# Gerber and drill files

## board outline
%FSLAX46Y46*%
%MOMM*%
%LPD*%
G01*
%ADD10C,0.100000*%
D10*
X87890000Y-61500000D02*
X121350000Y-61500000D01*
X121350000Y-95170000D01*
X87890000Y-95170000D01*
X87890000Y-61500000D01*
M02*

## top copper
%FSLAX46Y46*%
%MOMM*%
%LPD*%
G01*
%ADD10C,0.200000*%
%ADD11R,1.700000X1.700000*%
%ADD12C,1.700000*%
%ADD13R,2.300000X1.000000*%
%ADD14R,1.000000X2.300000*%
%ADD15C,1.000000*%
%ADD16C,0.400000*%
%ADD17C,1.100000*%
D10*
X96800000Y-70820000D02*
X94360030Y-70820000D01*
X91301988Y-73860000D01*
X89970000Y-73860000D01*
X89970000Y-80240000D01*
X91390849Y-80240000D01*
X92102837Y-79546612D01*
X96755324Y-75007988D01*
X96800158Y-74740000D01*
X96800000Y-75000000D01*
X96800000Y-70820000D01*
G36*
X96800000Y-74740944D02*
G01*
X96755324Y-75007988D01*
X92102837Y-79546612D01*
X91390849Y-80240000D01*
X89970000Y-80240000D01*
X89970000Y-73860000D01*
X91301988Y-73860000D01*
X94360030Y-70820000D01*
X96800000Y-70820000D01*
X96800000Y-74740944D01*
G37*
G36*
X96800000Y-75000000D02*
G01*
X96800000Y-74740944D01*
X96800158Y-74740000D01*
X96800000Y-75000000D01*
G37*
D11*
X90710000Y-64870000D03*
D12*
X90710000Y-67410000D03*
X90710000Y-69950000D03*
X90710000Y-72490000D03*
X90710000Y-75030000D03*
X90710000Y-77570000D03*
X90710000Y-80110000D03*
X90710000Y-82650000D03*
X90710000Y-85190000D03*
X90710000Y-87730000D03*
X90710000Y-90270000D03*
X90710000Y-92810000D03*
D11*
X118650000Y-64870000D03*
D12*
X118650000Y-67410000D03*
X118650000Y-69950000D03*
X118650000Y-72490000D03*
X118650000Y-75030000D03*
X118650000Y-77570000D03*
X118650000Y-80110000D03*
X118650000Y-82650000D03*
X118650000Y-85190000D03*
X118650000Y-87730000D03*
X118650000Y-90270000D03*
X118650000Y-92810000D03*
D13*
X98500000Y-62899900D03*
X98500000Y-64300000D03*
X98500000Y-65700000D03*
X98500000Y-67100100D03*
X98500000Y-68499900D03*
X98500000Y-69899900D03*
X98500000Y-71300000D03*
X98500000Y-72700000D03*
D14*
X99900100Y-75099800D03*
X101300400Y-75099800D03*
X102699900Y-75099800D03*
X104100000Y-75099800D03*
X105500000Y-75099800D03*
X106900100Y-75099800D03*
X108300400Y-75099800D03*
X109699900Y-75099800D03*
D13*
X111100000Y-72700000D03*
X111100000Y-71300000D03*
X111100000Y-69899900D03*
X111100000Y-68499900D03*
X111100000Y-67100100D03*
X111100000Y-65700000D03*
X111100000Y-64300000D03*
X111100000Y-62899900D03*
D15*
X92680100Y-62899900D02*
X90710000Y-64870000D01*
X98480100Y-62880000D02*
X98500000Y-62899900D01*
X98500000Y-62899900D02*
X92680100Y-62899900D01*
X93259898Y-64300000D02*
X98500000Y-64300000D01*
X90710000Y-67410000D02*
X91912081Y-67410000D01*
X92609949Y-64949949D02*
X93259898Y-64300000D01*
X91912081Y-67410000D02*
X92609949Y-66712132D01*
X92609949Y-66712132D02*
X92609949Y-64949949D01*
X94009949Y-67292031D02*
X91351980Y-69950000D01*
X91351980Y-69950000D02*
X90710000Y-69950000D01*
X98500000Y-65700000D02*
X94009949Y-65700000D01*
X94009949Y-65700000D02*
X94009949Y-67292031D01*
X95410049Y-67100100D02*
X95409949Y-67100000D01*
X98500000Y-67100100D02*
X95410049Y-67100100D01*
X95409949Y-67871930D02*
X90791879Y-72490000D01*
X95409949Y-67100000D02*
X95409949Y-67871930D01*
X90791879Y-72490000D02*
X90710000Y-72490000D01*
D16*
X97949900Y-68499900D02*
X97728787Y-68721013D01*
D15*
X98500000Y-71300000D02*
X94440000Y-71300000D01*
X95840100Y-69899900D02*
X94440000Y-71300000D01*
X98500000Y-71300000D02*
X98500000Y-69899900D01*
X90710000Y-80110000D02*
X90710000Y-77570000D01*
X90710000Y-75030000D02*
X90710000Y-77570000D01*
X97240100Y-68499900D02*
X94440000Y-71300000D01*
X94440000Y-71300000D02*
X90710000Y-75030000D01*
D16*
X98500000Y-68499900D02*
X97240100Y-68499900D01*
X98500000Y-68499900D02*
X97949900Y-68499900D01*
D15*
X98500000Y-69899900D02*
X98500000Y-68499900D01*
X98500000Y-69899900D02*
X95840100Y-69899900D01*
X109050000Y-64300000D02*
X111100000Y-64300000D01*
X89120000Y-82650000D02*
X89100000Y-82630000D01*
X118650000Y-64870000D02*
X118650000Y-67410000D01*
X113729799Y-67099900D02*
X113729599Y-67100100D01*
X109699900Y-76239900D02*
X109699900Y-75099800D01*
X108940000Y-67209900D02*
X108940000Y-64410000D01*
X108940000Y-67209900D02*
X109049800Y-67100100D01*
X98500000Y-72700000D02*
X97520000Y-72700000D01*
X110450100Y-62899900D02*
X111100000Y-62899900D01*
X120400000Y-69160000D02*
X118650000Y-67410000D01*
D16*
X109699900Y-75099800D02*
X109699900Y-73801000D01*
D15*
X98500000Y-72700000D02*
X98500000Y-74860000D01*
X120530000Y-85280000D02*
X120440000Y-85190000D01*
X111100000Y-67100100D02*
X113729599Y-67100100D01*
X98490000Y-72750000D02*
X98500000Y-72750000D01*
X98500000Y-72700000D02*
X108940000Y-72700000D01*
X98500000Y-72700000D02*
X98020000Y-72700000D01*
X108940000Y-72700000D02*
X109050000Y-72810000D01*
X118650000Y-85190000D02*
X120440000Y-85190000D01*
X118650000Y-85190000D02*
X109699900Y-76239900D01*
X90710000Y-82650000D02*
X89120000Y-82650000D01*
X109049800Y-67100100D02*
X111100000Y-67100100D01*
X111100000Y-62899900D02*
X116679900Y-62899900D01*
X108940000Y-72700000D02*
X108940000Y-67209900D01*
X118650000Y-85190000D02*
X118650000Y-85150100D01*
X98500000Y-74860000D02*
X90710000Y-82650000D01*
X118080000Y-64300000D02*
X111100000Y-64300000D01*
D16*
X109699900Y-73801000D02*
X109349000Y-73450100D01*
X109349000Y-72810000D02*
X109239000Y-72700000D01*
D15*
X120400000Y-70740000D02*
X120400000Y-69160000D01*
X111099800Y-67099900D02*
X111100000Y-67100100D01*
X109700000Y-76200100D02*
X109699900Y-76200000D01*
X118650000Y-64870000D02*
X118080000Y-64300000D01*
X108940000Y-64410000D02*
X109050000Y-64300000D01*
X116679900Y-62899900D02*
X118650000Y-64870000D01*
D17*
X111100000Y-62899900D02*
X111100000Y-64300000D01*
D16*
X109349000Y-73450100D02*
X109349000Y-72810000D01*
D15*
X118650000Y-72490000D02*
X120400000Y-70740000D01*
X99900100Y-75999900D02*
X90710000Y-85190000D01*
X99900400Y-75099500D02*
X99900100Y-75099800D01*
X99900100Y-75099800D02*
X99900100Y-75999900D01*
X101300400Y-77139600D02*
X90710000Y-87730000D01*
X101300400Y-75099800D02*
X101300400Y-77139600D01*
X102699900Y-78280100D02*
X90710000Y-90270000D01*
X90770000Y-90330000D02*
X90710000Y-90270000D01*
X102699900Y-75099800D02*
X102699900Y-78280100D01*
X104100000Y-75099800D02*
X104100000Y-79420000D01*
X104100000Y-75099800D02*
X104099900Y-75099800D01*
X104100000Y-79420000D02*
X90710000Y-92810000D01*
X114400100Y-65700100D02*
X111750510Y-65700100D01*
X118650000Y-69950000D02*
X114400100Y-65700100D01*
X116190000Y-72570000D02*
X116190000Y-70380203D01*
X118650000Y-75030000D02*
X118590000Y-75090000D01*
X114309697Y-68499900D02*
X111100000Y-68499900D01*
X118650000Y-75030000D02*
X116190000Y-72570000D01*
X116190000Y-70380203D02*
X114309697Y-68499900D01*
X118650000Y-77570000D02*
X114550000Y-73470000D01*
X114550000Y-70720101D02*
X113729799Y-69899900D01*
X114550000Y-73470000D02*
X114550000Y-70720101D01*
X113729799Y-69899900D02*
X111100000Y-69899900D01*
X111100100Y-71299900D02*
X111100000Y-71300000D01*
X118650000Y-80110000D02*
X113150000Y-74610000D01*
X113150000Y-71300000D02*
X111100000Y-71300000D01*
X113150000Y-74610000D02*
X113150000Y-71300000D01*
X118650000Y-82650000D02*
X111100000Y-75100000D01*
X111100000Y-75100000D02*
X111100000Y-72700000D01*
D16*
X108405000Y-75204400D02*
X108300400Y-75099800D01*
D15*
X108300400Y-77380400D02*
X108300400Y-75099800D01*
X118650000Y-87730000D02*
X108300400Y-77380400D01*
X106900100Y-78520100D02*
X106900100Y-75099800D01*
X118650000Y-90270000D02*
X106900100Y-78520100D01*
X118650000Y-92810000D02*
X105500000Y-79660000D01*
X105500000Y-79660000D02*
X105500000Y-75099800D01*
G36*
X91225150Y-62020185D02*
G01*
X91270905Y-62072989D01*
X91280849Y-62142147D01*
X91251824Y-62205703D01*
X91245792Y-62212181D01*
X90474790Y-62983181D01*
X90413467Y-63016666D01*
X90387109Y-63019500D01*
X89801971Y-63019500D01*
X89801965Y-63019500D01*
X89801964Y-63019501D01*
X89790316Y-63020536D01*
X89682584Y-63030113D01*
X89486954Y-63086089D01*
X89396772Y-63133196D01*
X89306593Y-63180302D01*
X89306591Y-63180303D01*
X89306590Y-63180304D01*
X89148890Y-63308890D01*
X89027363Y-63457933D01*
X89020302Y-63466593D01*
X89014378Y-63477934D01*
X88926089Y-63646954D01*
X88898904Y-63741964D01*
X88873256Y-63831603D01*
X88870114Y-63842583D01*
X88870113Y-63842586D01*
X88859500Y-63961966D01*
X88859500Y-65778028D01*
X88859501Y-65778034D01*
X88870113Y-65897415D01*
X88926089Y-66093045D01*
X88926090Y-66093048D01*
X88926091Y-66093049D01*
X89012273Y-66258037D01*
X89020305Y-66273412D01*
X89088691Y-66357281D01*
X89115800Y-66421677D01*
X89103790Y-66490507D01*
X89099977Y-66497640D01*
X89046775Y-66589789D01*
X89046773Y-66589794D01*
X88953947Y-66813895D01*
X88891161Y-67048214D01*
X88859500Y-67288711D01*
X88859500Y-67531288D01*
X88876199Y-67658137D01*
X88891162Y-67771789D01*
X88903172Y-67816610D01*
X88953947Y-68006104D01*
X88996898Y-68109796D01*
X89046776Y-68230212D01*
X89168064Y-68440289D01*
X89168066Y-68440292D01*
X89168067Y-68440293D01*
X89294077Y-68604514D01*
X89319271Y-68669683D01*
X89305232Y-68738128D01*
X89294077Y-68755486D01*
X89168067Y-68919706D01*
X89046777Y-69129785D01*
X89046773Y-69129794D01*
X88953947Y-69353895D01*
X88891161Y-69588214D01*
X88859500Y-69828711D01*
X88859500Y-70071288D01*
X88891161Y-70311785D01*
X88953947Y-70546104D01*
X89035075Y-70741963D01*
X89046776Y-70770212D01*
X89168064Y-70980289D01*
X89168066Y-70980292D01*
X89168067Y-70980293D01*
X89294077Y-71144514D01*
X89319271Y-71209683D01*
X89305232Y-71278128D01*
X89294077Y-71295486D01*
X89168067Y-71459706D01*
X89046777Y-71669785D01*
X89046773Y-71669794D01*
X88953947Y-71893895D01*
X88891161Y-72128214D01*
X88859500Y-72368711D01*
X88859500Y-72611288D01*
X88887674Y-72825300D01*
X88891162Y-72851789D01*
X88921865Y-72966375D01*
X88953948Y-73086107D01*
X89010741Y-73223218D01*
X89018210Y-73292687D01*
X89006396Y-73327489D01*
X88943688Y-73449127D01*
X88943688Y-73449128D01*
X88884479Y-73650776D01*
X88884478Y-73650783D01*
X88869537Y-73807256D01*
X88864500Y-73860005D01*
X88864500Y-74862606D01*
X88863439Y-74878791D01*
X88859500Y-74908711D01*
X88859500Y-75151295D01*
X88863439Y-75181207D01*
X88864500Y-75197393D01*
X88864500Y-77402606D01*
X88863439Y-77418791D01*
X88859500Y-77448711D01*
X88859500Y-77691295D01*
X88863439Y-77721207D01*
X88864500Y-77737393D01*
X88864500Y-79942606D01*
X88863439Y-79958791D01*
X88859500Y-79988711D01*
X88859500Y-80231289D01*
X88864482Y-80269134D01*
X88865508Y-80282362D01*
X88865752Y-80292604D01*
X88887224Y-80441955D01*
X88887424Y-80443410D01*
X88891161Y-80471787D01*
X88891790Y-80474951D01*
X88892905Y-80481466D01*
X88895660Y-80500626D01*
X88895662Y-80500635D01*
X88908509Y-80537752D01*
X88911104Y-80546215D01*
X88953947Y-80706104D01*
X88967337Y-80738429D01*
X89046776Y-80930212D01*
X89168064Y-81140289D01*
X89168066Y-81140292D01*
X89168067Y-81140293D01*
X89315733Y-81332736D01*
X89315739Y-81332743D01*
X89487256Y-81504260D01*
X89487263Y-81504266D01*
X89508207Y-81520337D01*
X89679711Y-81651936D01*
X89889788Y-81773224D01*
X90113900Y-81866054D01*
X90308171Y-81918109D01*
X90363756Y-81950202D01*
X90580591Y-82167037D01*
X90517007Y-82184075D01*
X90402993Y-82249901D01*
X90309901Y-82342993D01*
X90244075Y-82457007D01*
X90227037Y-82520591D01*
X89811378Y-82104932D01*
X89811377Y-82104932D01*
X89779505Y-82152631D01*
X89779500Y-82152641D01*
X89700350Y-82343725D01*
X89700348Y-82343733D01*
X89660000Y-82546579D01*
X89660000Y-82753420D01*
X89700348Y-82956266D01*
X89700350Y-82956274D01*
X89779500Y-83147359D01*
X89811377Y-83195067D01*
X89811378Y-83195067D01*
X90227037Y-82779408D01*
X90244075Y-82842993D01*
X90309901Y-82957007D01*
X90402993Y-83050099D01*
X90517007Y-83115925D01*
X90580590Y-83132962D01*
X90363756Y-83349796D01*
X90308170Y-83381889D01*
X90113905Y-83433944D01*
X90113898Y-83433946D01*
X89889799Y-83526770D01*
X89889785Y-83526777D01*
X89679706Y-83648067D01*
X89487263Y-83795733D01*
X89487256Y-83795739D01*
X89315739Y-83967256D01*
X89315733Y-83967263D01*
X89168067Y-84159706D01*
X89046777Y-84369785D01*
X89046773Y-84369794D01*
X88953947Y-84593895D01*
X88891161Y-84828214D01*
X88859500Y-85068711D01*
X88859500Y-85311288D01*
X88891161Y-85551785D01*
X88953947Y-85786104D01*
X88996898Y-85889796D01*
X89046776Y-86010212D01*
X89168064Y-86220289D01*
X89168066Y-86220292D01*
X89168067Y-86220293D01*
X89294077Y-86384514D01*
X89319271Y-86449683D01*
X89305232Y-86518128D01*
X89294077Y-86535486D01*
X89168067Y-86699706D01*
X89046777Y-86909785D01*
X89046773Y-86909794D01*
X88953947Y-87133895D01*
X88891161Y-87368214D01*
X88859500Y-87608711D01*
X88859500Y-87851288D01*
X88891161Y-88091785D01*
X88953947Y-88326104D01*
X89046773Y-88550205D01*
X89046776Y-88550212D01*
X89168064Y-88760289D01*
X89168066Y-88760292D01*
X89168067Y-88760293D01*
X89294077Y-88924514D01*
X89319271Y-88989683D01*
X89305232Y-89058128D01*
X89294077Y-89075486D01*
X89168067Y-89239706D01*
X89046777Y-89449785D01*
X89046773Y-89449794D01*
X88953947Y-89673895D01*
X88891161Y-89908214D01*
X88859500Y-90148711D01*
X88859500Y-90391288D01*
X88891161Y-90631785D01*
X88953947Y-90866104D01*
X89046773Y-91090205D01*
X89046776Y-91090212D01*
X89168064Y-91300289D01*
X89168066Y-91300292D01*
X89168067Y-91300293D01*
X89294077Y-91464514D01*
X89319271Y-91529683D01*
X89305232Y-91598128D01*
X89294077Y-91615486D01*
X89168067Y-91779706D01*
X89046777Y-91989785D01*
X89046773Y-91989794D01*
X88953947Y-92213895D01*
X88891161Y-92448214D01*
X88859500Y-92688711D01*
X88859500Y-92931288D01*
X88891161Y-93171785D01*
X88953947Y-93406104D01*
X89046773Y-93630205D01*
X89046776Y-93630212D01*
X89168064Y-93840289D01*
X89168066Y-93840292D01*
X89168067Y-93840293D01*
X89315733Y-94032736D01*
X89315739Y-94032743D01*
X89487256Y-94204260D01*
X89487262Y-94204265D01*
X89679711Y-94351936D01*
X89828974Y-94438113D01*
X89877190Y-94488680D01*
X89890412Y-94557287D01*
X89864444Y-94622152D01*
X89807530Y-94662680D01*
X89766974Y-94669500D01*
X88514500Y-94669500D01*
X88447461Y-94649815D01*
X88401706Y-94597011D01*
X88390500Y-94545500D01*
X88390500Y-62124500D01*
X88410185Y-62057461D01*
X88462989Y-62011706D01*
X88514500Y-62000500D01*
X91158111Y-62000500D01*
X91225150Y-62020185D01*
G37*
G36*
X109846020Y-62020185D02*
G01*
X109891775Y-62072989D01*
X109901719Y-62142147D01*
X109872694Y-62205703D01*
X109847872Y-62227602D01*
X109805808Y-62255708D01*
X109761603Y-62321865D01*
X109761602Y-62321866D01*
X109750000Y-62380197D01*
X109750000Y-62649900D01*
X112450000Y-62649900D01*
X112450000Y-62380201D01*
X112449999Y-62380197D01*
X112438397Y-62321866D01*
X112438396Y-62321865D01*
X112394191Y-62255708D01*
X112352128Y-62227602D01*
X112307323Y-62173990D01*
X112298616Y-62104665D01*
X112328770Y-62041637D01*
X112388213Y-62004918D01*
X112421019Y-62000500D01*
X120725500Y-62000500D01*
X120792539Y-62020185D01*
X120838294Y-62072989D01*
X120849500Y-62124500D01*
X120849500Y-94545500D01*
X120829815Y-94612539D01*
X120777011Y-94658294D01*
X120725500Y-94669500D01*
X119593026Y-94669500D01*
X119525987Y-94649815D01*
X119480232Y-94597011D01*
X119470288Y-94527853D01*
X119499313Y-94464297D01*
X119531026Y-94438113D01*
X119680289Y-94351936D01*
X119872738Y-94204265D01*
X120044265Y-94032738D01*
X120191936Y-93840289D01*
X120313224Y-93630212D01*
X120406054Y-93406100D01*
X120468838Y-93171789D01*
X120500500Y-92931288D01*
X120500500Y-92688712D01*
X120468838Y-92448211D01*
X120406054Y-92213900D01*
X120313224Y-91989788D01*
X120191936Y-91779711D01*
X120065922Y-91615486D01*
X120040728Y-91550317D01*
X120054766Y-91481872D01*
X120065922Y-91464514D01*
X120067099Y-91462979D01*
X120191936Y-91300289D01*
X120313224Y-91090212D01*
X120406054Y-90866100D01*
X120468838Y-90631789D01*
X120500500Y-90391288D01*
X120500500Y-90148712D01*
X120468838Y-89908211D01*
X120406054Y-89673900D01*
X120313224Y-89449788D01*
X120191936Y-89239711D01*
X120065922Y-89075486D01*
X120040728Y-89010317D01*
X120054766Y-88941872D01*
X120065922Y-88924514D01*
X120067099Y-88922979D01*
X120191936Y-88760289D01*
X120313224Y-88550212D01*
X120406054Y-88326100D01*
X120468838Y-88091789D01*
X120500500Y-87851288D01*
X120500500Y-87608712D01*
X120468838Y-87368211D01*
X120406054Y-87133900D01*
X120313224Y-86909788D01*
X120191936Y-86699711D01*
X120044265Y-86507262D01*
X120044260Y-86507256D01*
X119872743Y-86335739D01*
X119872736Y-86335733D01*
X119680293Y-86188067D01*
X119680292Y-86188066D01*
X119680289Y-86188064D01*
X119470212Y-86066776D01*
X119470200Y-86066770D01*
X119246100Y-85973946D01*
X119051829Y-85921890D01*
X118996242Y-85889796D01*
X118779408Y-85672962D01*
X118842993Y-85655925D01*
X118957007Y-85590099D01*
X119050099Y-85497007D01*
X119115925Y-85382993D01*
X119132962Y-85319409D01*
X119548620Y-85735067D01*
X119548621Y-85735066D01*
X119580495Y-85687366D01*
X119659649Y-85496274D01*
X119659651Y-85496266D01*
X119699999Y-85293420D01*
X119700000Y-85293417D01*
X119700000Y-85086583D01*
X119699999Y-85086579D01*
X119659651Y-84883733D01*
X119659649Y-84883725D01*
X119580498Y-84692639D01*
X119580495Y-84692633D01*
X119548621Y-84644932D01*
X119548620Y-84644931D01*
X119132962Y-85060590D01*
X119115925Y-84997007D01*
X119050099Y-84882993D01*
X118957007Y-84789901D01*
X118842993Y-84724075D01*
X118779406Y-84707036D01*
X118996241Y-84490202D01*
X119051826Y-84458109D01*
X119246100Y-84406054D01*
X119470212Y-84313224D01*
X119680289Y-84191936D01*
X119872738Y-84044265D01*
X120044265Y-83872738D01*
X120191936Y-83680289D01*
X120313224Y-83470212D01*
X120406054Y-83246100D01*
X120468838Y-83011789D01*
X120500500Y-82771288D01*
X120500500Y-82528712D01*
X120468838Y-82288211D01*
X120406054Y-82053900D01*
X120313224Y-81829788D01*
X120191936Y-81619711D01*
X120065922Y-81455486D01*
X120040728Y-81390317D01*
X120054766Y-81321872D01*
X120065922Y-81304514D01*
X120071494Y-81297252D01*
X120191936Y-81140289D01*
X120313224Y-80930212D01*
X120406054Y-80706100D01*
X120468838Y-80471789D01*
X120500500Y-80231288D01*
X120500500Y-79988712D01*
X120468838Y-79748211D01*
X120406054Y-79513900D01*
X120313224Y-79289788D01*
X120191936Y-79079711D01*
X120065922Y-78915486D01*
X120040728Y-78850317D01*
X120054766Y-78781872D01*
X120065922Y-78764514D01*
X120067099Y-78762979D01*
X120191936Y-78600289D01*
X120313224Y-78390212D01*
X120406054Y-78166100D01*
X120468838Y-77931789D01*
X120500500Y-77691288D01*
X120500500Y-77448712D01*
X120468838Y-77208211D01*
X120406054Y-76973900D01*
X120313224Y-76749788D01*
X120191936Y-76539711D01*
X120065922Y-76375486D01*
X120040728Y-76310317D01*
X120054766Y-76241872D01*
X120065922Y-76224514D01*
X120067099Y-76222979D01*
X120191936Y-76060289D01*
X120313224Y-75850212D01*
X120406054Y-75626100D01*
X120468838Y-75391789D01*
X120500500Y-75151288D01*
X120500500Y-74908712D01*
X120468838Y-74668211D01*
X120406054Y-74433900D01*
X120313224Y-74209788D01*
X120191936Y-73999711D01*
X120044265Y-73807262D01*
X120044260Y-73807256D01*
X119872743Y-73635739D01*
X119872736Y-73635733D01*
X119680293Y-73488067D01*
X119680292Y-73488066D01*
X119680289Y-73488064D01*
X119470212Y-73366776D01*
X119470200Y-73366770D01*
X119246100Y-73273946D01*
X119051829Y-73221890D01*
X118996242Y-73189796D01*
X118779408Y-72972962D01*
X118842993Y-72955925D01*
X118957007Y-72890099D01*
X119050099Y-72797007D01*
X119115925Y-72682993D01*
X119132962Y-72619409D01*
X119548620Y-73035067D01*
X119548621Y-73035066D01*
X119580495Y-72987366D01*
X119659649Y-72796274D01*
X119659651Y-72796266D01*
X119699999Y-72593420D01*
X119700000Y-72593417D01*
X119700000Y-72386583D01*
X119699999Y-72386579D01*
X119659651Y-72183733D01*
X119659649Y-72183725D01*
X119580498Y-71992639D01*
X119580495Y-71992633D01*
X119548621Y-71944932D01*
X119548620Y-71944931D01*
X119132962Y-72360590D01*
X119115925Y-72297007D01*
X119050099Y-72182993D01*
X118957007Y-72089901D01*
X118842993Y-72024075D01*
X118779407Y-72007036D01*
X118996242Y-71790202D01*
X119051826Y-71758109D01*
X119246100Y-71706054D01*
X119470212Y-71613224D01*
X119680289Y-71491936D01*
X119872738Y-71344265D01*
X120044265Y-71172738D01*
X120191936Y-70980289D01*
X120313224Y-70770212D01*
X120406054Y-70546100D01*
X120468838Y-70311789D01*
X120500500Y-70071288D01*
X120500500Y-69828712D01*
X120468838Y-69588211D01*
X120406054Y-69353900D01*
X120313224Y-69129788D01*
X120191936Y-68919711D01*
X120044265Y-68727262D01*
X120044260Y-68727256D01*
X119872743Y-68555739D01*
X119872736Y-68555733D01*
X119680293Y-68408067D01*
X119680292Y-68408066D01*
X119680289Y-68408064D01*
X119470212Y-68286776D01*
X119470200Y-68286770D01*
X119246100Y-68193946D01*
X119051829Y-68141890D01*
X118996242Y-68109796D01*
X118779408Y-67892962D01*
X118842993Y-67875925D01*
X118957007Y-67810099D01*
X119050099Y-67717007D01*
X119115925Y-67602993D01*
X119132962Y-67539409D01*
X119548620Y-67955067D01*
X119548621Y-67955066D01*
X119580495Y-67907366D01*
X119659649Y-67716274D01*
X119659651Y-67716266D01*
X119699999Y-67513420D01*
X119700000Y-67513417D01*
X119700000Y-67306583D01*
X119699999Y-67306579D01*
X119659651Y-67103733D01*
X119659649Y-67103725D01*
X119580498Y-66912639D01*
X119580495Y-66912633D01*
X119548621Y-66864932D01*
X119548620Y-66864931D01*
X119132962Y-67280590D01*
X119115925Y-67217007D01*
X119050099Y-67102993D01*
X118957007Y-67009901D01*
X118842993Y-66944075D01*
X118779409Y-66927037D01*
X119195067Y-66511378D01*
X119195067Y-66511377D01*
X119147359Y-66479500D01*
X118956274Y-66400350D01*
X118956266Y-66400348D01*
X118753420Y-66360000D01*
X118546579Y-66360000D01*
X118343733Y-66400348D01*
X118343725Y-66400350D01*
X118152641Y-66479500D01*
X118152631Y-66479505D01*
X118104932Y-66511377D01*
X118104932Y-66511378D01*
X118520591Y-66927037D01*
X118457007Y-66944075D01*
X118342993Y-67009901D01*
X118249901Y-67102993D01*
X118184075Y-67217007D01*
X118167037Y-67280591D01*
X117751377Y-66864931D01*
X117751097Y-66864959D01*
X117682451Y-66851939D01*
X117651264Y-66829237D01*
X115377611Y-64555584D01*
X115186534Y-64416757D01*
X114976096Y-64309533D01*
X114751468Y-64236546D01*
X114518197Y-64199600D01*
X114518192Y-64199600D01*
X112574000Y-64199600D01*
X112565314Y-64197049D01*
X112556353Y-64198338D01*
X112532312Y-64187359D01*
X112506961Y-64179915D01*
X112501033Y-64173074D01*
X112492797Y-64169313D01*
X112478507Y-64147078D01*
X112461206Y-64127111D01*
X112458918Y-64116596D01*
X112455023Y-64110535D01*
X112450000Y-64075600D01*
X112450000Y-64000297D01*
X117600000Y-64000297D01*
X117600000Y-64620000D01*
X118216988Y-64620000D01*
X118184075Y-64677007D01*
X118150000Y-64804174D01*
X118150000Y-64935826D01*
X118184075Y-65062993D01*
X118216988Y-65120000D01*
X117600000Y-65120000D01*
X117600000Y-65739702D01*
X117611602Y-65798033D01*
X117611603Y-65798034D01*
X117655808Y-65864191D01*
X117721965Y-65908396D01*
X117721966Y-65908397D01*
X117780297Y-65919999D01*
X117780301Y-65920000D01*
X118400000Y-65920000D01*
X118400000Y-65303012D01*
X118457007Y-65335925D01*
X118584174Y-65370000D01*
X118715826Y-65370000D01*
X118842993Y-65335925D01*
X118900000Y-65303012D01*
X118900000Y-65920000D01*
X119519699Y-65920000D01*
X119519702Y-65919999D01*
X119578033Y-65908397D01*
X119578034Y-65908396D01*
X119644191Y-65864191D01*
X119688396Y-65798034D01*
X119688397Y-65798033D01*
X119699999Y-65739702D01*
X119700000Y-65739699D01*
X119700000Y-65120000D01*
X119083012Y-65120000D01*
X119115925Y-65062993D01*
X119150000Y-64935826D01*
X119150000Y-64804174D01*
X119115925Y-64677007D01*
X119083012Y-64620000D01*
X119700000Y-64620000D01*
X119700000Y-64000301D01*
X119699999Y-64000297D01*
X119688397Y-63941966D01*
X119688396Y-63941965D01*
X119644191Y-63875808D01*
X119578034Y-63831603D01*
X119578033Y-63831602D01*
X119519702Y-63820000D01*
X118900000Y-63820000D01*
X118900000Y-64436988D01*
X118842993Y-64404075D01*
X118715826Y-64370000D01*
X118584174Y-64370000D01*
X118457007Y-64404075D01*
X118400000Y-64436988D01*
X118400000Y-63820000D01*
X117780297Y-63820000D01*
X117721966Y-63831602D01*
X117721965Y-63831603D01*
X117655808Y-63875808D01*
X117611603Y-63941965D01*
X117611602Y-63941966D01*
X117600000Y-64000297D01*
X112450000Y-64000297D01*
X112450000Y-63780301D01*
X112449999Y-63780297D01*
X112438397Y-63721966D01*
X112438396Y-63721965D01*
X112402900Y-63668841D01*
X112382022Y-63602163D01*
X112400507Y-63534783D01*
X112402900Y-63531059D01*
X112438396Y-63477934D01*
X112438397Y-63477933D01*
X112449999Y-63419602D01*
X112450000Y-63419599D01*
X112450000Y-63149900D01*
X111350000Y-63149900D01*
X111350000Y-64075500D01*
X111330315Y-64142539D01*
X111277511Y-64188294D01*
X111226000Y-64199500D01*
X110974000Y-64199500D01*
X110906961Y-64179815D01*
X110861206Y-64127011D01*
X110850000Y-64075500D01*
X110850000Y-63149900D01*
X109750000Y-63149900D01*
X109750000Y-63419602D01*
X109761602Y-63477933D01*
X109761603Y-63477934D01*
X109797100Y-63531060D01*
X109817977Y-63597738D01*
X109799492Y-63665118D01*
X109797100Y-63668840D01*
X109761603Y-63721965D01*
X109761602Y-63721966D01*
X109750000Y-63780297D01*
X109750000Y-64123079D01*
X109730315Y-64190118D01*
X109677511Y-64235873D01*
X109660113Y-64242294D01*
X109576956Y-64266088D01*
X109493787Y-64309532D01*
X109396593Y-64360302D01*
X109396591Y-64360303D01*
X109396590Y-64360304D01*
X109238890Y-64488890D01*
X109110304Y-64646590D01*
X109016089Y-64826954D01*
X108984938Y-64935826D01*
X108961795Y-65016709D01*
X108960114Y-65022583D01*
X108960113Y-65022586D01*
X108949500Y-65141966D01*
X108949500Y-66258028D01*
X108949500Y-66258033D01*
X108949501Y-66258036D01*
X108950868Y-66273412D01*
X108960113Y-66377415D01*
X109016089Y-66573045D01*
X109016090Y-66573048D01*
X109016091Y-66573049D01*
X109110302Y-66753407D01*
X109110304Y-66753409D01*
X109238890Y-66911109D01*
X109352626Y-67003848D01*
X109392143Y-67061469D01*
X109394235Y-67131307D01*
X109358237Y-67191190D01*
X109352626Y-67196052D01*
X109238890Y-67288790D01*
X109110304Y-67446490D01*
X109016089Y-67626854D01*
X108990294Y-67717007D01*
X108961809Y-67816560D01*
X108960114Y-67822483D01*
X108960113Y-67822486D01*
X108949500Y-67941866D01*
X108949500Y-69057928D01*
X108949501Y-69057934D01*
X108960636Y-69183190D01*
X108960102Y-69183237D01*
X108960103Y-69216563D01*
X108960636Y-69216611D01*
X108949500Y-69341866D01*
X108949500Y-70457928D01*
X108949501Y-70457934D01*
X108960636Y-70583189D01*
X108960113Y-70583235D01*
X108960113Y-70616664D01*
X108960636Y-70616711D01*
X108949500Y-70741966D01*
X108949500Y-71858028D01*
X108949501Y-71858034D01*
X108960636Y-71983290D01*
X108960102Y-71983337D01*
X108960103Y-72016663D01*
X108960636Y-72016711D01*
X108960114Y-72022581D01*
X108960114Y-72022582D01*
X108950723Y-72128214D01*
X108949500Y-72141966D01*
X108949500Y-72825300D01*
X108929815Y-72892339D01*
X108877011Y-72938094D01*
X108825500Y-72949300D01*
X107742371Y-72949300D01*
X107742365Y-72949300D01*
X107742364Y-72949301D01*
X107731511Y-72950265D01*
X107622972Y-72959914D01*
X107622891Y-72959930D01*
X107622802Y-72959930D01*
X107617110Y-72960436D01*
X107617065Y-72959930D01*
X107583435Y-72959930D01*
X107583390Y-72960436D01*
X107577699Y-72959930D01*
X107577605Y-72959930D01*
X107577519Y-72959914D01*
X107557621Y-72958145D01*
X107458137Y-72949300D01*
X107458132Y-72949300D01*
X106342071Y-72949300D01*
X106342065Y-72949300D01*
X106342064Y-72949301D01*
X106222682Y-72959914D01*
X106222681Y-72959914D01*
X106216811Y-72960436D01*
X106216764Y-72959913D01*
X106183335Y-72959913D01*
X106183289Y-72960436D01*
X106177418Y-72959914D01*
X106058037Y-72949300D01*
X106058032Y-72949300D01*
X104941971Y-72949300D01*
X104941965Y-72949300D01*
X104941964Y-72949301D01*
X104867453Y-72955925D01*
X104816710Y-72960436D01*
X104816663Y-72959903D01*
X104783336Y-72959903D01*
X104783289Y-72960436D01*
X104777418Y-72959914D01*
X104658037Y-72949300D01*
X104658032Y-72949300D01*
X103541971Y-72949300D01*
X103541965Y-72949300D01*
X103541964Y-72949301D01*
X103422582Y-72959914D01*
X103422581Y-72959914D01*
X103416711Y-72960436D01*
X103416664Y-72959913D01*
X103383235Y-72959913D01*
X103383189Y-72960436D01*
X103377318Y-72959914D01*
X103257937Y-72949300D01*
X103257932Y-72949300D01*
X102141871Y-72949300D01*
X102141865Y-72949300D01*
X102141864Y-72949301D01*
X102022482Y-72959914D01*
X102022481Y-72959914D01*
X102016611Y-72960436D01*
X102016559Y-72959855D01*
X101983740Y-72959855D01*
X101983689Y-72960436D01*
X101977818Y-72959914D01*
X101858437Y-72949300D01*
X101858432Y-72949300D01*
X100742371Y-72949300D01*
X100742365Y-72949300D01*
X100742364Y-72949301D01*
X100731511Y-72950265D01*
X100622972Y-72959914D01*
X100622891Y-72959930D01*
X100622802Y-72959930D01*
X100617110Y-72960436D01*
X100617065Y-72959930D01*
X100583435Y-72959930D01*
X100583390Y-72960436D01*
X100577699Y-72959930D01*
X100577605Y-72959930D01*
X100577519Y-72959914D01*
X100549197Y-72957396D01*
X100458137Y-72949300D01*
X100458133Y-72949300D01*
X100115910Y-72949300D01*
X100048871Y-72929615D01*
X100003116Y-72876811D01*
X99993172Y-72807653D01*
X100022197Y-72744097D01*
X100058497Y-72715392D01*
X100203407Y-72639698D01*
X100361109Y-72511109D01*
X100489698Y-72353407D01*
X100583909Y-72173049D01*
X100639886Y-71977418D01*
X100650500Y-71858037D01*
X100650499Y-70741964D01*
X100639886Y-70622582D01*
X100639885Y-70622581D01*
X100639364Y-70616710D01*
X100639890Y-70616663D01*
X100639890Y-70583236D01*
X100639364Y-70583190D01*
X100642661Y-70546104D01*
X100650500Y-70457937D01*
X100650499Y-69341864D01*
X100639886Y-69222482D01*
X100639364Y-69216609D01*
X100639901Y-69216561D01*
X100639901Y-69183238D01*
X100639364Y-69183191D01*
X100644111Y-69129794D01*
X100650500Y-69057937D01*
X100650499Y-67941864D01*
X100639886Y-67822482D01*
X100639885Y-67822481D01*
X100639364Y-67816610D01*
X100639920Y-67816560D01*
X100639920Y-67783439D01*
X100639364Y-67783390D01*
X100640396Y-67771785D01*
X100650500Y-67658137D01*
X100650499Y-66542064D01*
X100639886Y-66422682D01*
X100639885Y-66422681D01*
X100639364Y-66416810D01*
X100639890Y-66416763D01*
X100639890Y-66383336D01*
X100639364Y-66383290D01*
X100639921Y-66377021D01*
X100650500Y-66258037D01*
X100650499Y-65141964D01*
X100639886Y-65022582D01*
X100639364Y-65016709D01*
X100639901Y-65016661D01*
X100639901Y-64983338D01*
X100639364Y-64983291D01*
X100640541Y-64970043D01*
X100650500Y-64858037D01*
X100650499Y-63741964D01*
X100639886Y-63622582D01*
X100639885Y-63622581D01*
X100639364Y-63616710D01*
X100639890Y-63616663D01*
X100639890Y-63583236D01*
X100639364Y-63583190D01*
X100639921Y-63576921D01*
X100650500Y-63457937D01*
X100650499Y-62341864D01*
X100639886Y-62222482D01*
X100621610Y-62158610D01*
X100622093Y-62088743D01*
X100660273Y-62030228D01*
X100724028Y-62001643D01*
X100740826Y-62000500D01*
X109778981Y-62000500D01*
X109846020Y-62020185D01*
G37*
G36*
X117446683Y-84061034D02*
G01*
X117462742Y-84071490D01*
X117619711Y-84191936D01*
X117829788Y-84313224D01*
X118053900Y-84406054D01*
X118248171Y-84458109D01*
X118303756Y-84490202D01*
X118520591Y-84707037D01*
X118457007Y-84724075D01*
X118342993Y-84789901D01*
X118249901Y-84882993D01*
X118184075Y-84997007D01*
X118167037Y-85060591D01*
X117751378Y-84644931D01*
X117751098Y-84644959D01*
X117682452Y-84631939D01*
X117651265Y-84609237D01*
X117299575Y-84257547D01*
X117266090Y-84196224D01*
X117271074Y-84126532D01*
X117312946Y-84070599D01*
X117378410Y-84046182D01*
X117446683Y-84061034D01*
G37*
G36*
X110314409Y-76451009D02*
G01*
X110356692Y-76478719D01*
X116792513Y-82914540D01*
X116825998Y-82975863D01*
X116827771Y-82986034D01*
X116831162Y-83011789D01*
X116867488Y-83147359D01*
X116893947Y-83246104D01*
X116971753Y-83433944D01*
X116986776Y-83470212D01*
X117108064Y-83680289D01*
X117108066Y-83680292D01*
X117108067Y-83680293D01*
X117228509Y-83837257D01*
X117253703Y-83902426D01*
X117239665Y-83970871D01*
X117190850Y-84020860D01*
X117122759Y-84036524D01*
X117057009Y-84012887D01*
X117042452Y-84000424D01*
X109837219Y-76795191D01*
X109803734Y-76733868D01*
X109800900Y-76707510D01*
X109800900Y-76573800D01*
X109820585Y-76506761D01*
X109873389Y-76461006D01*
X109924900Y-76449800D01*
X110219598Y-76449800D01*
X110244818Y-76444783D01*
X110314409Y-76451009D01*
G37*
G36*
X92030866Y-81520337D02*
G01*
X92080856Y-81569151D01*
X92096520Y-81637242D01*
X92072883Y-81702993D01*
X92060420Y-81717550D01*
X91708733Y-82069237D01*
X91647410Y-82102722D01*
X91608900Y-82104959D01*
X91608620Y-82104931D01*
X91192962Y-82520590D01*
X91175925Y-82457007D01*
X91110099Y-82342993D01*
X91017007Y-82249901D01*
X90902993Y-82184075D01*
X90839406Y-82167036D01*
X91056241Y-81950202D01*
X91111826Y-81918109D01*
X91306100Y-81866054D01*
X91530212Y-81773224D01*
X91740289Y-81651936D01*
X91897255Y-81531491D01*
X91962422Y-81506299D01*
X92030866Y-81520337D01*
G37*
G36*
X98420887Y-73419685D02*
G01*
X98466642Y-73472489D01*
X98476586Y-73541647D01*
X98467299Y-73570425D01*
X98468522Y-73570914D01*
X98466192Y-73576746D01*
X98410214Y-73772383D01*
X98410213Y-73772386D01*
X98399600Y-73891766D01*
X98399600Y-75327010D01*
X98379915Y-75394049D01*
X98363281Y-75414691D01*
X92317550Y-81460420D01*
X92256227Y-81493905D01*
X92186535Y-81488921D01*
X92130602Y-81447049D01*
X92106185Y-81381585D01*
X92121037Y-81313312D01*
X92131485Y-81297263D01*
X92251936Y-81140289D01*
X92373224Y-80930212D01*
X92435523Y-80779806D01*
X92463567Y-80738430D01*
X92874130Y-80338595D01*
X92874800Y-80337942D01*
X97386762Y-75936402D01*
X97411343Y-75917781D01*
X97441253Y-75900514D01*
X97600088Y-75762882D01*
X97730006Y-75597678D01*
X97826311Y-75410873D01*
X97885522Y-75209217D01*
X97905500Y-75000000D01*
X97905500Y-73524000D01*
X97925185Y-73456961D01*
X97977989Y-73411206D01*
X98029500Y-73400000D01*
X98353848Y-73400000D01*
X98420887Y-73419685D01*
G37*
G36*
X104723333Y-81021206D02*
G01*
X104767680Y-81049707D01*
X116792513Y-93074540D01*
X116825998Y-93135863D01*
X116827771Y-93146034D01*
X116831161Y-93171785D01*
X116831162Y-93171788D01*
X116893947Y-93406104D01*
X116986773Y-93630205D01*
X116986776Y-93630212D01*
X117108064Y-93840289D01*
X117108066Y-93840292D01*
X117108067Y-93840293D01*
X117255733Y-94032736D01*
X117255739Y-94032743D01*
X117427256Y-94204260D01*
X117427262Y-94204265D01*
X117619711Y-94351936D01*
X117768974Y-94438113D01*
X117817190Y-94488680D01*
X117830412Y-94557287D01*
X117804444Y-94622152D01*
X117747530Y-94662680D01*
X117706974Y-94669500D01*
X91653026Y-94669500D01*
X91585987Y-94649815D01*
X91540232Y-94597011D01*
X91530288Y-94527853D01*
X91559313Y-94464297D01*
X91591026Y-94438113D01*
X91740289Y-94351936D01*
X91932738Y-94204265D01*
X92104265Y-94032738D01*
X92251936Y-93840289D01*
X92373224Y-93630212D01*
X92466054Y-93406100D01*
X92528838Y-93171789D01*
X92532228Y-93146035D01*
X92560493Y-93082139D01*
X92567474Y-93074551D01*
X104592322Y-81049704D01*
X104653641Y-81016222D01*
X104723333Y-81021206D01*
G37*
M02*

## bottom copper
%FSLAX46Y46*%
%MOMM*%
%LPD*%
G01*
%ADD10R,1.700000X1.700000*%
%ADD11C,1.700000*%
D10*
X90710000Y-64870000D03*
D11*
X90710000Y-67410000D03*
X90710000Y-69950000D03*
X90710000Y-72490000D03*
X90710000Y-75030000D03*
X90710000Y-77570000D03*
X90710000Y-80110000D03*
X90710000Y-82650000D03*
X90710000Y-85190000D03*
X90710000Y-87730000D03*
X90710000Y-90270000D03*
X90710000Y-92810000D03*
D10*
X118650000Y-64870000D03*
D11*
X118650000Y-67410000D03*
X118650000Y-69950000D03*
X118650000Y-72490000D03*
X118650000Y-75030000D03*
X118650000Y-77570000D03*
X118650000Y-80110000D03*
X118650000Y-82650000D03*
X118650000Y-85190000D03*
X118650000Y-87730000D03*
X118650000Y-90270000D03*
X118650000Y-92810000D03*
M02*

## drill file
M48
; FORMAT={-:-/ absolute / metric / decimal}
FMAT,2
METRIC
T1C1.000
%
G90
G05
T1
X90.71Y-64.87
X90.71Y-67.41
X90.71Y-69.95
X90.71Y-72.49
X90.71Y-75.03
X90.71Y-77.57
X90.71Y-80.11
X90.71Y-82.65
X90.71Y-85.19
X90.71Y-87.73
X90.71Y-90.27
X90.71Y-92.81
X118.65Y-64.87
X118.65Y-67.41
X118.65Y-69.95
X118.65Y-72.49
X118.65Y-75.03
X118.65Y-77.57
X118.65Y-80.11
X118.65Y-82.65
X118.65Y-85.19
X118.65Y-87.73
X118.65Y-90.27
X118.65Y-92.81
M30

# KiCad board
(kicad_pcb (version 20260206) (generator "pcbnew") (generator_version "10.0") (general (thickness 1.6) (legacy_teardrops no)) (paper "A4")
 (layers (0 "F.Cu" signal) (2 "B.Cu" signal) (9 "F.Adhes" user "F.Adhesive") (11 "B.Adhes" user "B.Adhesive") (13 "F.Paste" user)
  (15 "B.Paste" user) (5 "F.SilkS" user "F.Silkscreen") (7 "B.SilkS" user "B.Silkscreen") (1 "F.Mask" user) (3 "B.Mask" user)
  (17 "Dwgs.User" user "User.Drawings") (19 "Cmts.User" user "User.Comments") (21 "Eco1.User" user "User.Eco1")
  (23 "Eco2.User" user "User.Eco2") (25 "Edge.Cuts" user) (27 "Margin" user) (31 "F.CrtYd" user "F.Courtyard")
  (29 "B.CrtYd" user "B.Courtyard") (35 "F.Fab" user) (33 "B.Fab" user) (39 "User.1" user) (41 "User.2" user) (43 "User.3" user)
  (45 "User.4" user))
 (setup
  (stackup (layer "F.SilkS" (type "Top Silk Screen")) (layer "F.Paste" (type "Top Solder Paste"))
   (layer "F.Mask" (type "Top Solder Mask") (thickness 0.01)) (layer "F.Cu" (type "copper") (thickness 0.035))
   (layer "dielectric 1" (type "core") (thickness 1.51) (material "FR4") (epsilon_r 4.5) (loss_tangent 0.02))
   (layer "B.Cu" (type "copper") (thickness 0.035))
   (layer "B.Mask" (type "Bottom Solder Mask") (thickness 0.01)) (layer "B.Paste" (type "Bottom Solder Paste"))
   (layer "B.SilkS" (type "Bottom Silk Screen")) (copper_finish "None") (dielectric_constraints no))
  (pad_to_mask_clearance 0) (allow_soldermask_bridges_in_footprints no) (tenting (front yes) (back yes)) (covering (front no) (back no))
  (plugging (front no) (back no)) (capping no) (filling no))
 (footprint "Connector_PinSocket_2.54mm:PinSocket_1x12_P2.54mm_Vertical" (layer "F.Cu") (at 90.71 64.87)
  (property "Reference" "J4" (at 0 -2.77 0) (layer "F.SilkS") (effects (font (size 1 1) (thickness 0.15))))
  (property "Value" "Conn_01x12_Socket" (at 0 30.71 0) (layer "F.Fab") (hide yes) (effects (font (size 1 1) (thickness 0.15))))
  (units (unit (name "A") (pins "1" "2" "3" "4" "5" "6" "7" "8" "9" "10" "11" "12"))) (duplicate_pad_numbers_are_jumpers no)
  (pad "1" thru_hole rect (at 0 0) (size 1.7 1.7) (drill 1) (layers "*.Cu" "*.Mask") (remove_unused_layers no) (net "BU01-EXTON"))
  (pad "2" thru_hole circle (at 0 2.54) (size 1.7 1.7) (drill 1) (layers "*.Cu" "*.Mask") (remove_unused_layers no) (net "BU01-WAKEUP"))
  (pad "3" thru_hole circle (at 0 5.08) (size 1.7 1.7) (drill 1) (layers "*.Cu" "*.Mask") (remove_unused_layers no) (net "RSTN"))
  (pad "4" thru_hole circle (at 0 7.62) (size 1.7 1.7) (drill 1) (layers "*.Cu" "*.Mask") (remove_unused_layers no) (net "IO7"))
  (pad "5" thru_hole circle (at 0 10.16) (size 1.7 1.7) (drill 1) (layers "*.Cu" "*.Mask") (remove_unused_layers no) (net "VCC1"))
  (pad "6" thru_hole circle (at 0 12.7) (size 1.7 1.7) (drill 1) (layers "*.Cu" "*.Mask") (remove_unused_layers no) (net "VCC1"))
  (pad "7" thru_hole circle (at 0 15.24) (size 1.7 1.7) (drill 1) (layers "*.Cu" "*.Mask") (remove_unused_layers no) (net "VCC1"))
  (pad "8" thru_hole circle (at 0 17.78) (size 1.7 1.7) (drill 1) (layers "*.Cu" "*.Mask") (remove_unused_layers no) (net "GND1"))
  (pad "9" thru_hole circle (at 0 20.32) (size 1.7 1.7) (drill 1) (layers "*.Cu" "*.Mask") (remove_unused_layers no) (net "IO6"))
  (pad "10" thru_hole circle (at 0 22.86) (size 1.7 1.7) (drill 1) (layers "*.Cu" "*.Mask") (remove_unused_layers no) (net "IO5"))
  (pad "11" thru_hole circle (at 0 25.4) (size 1.7 1.7) (drill 1) (layers "*.Cu" "*.Mask") (remove_unused_layers no) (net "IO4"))
  (pad "12" thru_hole circle (at 0 27.94) (size 1.7 1.7) (drill 1) (layers "*.Cu" "*.Mask") (remove_unused_layers no) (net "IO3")))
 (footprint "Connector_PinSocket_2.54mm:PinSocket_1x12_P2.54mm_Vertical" (layer "F.Cu") (at 118.65 64.87)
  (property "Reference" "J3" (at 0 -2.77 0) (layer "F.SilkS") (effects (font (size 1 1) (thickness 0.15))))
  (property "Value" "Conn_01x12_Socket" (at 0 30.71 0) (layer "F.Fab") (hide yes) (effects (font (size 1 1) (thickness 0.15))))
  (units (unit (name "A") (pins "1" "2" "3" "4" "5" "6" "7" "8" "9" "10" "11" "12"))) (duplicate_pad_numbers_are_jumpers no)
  (pad "1" thru_hole rect (at 0 0) (size 1.7 1.7) (drill 1) (layers "*.Cu" "*.Mask") (remove_unused_layers no) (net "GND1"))
  (pad "2" thru_hole circle (at 0 2.54) (size 1.7 1.7) (drill 1) (layers "*.Cu" "*.Mask") (remove_unused_layers no) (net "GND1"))
  (pad "3" thru_hole circle (at 0 5.08) (size 1.7 1.7) (drill 1) (layers "*.Cu" "*.Mask") (remove_unused_layers no) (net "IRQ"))
  (pad "4" thru_hole circle (at 0 7.62) (size 1.7 1.7) (drill 1) (layers "*.Cu" "*.Mask") (remove_unused_layers no) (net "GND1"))
  (pad "5" thru_hole circle (at 0 10.16) (size 1.7 1.7) (drill 1) (layers "*.Cu" "*.Mask") (remove_unused_layers no) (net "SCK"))
  (pad "6" thru_hole circle (at 0 12.7) (size 1.7 1.7) (drill 1) (layers "*.Cu" "*.Mask") (remove_unused_layers no) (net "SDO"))
  (pad "7" thru_hole circle (at 0 15.24) (size 1.7 1.7) (drill 1) (layers "*.Cu" "*.Mask") (remove_unused_layers no) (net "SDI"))
  (pad "8" thru_hole circle (at 0 17.78) (size 1.7 1.7) (drill 1) (layers "*.Cu" "*.Mask") (remove_unused_layers no) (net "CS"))
  (pad "9" thru_hole circle (at 0 20.32) (size 1.7 1.7) (drill 1) (layers "*.Cu" "*.Mask") (remove_unused_layers no) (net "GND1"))
  (pad "10" thru_hole circle (at 0 22.86) (size 1.7 1.7) (drill 1) (layers "*.Cu" "*.Mask") (remove_unused_layers no) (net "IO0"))
  (pad "11" thru_hole circle (at 0 25.4) (size 1.7 1.7) (drill 1) (layers "*.Cu" "*.Mask") (remove_unused_layers no) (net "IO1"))
  (pad "12" thru_hole circle (at 0 27.94) (size 1.7 1.7) (drill 1) (layers "*.Cu" "*.Mask") (remove_unused_layers no) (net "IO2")))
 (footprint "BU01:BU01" (layer "F.Cu") (at 104.8 69)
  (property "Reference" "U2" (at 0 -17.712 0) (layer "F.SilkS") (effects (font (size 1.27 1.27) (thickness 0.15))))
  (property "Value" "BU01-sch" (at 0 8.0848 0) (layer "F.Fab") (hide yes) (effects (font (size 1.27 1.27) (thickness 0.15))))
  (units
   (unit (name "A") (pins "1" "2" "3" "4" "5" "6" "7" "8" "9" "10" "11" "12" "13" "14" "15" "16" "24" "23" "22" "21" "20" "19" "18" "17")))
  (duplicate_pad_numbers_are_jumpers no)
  (pad "1" smd rect (at -6.3 -6.1001) (size 2.3 1) (layers "F.Cu" "F.Mask" "F.Paste") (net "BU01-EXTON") (solder_mask_margin 0.0508)
   (solder_paste_margin 0) (thermal_bridge_angle 0))
  (pad "2" smd rect (at -6.3 -4.7) (size 2.3 1) (layers "F.Cu" "F.Mask" "F.Paste") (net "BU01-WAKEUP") (solder_mask_margin 0.0508)
   (solder_paste_margin 0) (thermal_bridge_angle 0))
  (pad "3" smd rect (at -6.3 -3.3) (size 2.3 1) (layers "F.Cu" "F.Mask" "F.Paste") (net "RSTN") (solder_mask_margin 0.0508)
   (solder_paste_margin 0) (thermal_bridge_angle 0))
  (pad "4" smd rect (at -6.3 -1.8999) (size 2.3 1) (layers "F.Cu" "F.Mask" "F.Paste") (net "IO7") (solder_mask_margin 0.0508)
   (solder_paste_margin 0) (thermal_bridge_angle 0))
  (pad "5" smd rect (at -6.3 -0.5001) (size 2.3 1) (layers "F.Cu" "F.Mask" "F.Paste") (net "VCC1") (solder_mask_margin 0.0508)
   (solder_paste_margin 0) (thermal_bridge_angle 0))
  (pad "6" smd rect (at -6.3 0.8999) (size 2.3 1) (layers "F.Cu" "F.Mask" "F.Paste") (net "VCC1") (solder_mask_margin 0.0508)
   (solder_paste_margin 0) (thermal_bridge_angle 0))
  (pad "7" smd rect (at -6.3 2.3) (size 2.3 1) (layers "F.Cu" "F.Mask" "F.Paste") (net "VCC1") (solder_mask_margin 0.0508)
   (solder_paste_margin 0) (thermal_bridge_angle 0))
  (pad "8" smd rect (at -6.3 3.7) (size 2.3 1) (layers "F.Cu" "F.Mask" "F.Paste") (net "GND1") (solder_mask_margin 0.0508)
   (solder_paste_margin 0) (thermal_bridge_angle 0))
  (pad "9" smd rect (at -4.8999 6.0998) (size 1 2.3) (layers "F.Cu" "F.Mask" "F.Paste") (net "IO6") (solder_mask_margin 0.0508)
   (solder_paste_margin 0) (thermal_bridge_angle 0))
  (pad "10" smd rect (at -3.4996 6.0998) (size 1 2.3) (layers "F.Cu" "F.Mask" "F.Paste") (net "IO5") (solder_mask_margin 0.0508)
   (solder_paste_margin 0) (thermal_bridge_angle 0))
  (pad "11" smd rect (at -2.1001 6.0998) (size 1 2.3) (layers "F.Cu" "F.Mask" "F.Paste") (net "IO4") (solder_mask_margin 0.0508)
   (solder_paste_margin 0) (thermal_bridge_angle 0))
  (pad "12" smd rect (at -0.7 6.0998) (size 1 2.3) (layers "F.Cu" "F.Mask" "F.Paste") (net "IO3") (solder_mask_margin 0.0508)
   (solder_paste_margin 0) (thermal_bridge_angle 0))
  (pad "13" smd rect (at 0.7 6.0998) (size 1 2.3) (layers "F.Cu" "F.Mask" "F.Paste") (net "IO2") (solder_mask_margin 0.0508)
   (solder_paste_margin 0) (thermal_bridge_angle 0))
  (pad "14" smd rect (at 2.1001 6.0998) (size 1 2.3) (layers "F.Cu" "F.Mask" "F.Paste") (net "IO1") (solder_mask_margin 0.0508)
   (solder_paste_margin 0) (thermal_bridge_angle 0))
  (pad "15" smd rect (at 3.5004 6.0998) (size 1 2.3) (layers "F.Cu" "F.Mask" "F.Paste") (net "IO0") (solder_mask_margin 0.0508)
   (solder_paste_margin 0) (thermal_bridge_angle 0))
  (pad "16" smd rect (at 4.8999 6.0998) (size 1 2.3) (layers "F.Cu" "F.Mask" "F.Paste") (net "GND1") (solder_mask_margin 0.0508)
   (solder_paste_margin 0) (thermal_bridge_angle 0))
  (pad "17" smd rect (at 6.3 3.7) (size 2.3 1) (layers "F.Cu" "F.Mask" "F.Paste") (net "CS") (solder_mask_margin 0.0508)
   (solder_paste_margin 0) (thermal_bridge_angle 0))
  (pad "18" smd rect (at 6.3 2.3) (size 2.3 1) (layers "F.Cu" "F.Mask" "F.Paste") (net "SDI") (solder_mask_margin 0.0508)
   (solder_paste_margin 0) (thermal_bridge_angle 0))
  (pad "19" smd rect (at 6.3 0.8999) (size 2.3 1) (layers "F.Cu" "F.Mask" "F.Paste") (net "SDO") (solder_mask_margin 0.0508)
   (solder_paste_margin 0) (thermal_bridge_angle 0))
  (pad "20" smd rect (at 6.3 -0.5001) (size 2.3 1) (layers "F.Cu" "F.Mask" "F.Paste") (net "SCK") (solder_mask_margin 0.0508)
   (solder_paste_margin 0) (thermal_bridge_angle 0))
  (pad "21" smd rect (at 6.3 -1.8999) (size 2.3 1) (layers "F.Cu" "F.Mask" "F.Paste") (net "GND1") (solder_mask_margin 0.0508)
   (solder_paste_margin 0) (thermal_bridge_angle 0))
  (pad "22" smd rect (at 6.3 -3.3) (size 2.3 1) (layers "F.Cu" "F.Mask" "F.Paste") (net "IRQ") (solder_mask_margin 0.0508)
   (solder_paste_margin 0) (thermal_bridge_angle 0))
  (pad "23" smd rect (at 6.3 -4.7) (size 2.3 1) (layers "F.Cu" "F.Mask" "F.Paste") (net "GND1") (solder_mask_margin 0.0508)
   (solder_paste_margin 0) (thermal_bridge_angle 0))
  (pad "24" smd rect (at 6.3 -6.1001) (size 2.3 1) (layers "F.Cu" "F.Mask" "F.Paste") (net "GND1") (solder_mask_margin 0.0508)
   (solder_paste_margin 0) (thermal_bridge_angle 0)))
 (gr_poly
  (pts (xy 96.8 70.82) (xy 94.36003 70.82) (xy 91.301988 73.86) (xy 89.97 73.86) (xy 89.97 80.24) (xy 91.390849 80.24)
   (xy 92.102837 79.546612) (xy 96.755324 75.007988) (xy 96.800158 74.74) (xy 96.8 75))
  (stroke (width 0.2) (type solid)) (fill yes) (layer "F.Cu") (net "VCC1"))
 (gr_rect (start 87.89 61.5) (end 121.35 95.17) (stroke (width 0.1) (type solid)) (fill no) (layer "Edge.Cuts"))
 (segment (start 92.6801 62.8999) (end 90.71 64.87) (width 1) (layer "F.Cu") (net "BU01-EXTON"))
 (segment (start 98.4801 62.88) (end 98.5 62.8999) (width 1) (layer "F.Cu") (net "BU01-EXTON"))
 (segment (start 98.5 62.8999) (end 92.6801 62.8999) (width 1) (layer "F.Cu") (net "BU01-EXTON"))
 (segment (start 93.259898 64.3) (end 98.5 64.3) (width 1) (layer "F.Cu") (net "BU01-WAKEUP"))
 (segment (start 90.71 67.41) (end 91.912081 67.41) (width 1) (layer "F.Cu") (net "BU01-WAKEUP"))
 (segment (start 92.609949 64.949949) (end 93.259898 64.3) (width 1) (layer "F.Cu") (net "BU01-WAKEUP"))
 (segment (start 91.912081 67.41) (end 92.609949 66.712132) (width 1) (layer "F.Cu") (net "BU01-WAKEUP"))
 (segment (start 92.609949 66.712132) (end 92.609949 64.949949) (width 1) (layer "F.Cu") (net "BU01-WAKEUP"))
 (segment (start 94.009949 67.292031) (end 91.35198 69.95) (width 1) (layer "F.Cu") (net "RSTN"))
 (segment (start 91.35198 69.95) (end 90.71 69.95) (width 1) (layer "F.Cu") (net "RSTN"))
 (segment (start 98.5 65.7) (end 94.009949 65.7) (width 1) (layer "F.Cu") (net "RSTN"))
 (segment (start 94.009949 65.7) (end 94.009949 67.292031) (width 1) (layer "F.Cu") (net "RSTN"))
 (segment (start 95.410049 67.1001) (end 95.409949 67.1) (width 1) (layer "F.Cu") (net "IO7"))
 (segment (start 98.5 67.1001) (end 95.410049 67.1001) (width 1) (layer "F.Cu") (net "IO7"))
 (segment (start 95.409949 67.87193) (end 90.791879 72.49) (width 1) (layer "F.Cu") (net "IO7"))
 (segment (start 95.409949 67.1) (end 95.409949 67.87193) (width 1) (layer "F.Cu") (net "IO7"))
 (segment (start 90.791879 72.49) (end 90.71 72.49) (width 1) (layer "F.Cu") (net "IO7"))
 (segment (start 97.9499 68.4999) (end 97.728787 68.721013) (width 0.4) (layer "F.Cu") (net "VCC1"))
 (segment (start 98.5 71.3) (end 94.44 71.3) (width 1) (layer "F.Cu") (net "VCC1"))
 (segment (start 95.8401 69.8999) (end 94.44 71.3) (width 1) (layer "F.Cu") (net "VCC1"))
 (segment (start 98.5 71.3) (end 98.5 69.8999) (width 1) (layer "F.Cu") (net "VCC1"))
 (segment (start 90.71 80.11) (end 90.71 77.57) (width 1) (layer "F.Cu") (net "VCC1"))
 (segment (start 90.71 75.03) (end 90.71 77.57) (width 1) (layer "F.Cu") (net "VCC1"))
 (segment (start 97.2401 68.4999) (end 94.44 71.3) (width 1) (layer "F.Cu") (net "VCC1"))
 (segment (start 94.44 71.3) (end 90.71 75.03) (width 1) (layer "F.Cu") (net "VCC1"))
 (segment (start 98.5 68.4999) (end 97.2401 68.4999) (width 0.4) (layer "F.Cu") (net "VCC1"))
 (segment (start 98.5 68.4999) (end 97.9499 68.4999) (width 0.4) (layer "F.Cu") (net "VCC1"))
 (segment (start 98.5 69.8999) (end 98.5 68.4999) (width 1) (layer "F.Cu") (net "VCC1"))
 (segment (start 98.5 69.8999) (end 95.8401 69.8999) (width 1) (layer "F.Cu") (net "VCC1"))
 (segment (start 109.05 64.3) (end 111.1 64.3) (width 1) (layer "F.Cu") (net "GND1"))
 (segment (start 89.12 82.65) (end 89.1 82.63) (width 1) (layer "F.Cu") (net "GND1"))
 (segment (start 118.65 64.87) (end 118.65 67.41) (width 1) (layer "F.Cu") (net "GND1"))
 (segment (start 113.729799 67.0999) (end 113.729599 67.1001) (width 1) (layer "F.Cu") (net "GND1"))
 (segment (start 109.6999 76.2399) (end 109.6999 75.0998) (width 1) (layer "F.Cu") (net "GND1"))
 (segment (start 108.94 67.2099) (end 108.94 64.41) (width 1) (layer "F.Cu") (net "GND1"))
 (segment (start 108.94 67.2099) (end 109.0498 67.1001) (width 1) (layer "F.Cu") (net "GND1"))
 (segment (start 98.5 72.7) (end 97.52 72.7) (width 1) (layer "F.Cu") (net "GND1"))
 (segment (start 110.4501 62.8999) (end 111.1 62.8999) (width 1) (layer "F.Cu") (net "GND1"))
 (segment (start 120.4 69.16) (end 118.65 67.41) (width 1) (layer "F.Cu") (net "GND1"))
 (segment (start 109.6999 75.0998) (end 109.6999 73.801) (width 0.4) (layer "F.Cu") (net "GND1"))
 (segment (start 98.5 72.7) (end 98.5 74.86) (width 1) (layer "F.Cu") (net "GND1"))
 (segment (start 120.53 85.28) (end 120.44 85.19) (width 1) (layer "F.Cu") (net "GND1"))
 (segment (start 111.1 67.1001) (end 113.729599 67.1001) (width 1) (layer "F.Cu") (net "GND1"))
 (segment (start 98.49 72.75) (end 98.5 72.75) (width 1) (layer "F.Cu") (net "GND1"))
 (segment (start 98.5 72.7) (end 108.94 72.7) (width 1) (layer "F.Cu") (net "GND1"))
 (segment (start 98.5 72.7) (end 98.02 72.7) (width 1) (layer "F.Cu") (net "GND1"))
 (segment (start 108.94 72.7) (end 109.05 72.81) (width 1) (layer "F.Cu") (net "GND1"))
 (segment (start 118.65 85.19) (end 120.44 85.19) (width 1) (layer "F.Cu") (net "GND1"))
 (segment (start 118.65 85.19) (end 109.6999 76.2399) (width 1) (layer "F.Cu") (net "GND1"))
 (segment (start 90.71 82.65) (end 89.12 82.65) (width 1) (layer "F.Cu") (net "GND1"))
 (segment (start 109.0498 67.1001) (end 111.1 67.1001) (width 1) (layer "F.Cu") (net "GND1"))
 (segment (start 111.1 62.8999) (end 116.6799 62.8999) (width 1) (layer "F.Cu") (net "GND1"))
 (segment (start 108.94 72.7) (end 108.94 67.2099) (width 1) (layer "F.Cu") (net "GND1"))
 (segment (start 118.65 85.19) (end 118.65 85.1501) (width 1) (layer "F.Cu") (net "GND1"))
 (segment (start 98.5 74.86) (end 90.71 82.65) (width 1) (layer "F.Cu") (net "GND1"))
 (segment (start 118.08 64.3) (end 111.1 64.3) (width 1) (layer "F.Cu") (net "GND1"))
 (segment (start 109.6999 73.801) (end 109.349 73.4501) (width 0.4) (layer "F.Cu") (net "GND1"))
 (segment (start 109.349 72.81) (end 109.239 72.7) (width 0.4) (layer "F.Cu") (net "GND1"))
 (segment (start 120.4 70.74) (end 120.4 69.16) (width 1) (layer "F.Cu") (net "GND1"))
 (segment (start 111.0998 67.0999) (end 111.1 67.1001) (width 1) (layer "F.Cu") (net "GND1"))
 (segment (start 109.7 76.2001) (end 109.6999 76.2) (width 1) (layer "F.Cu") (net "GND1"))
 (segment (start 118.65 64.87) (end 118.08 64.3) (width 1) (layer "F.Cu") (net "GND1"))
 (segment (start 108.94 64.41) (end 109.05 64.3) (width 1) (layer "F.Cu") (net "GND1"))
 (segment (start 116.6799 62.8999) (end 118.65 64.87) (width 1) (layer "F.Cu") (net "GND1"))
 (segment (start 111.1 62.8999) (end 111.1 64.3) (width 1.1) (layer "F.Cu") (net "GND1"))
 (segment (start 109.349 73.4501) (end 109.349 72.81) (width 0.4) (layer "F.Cu") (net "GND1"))
 (segment (start 118.65 72.49) (end 120.4 70.74) (width 1) (layer "F.Cu") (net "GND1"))
 (segment (start 99.9001 75.9999) (end 90.71 85.19) (width 1) (layer "F.Cu") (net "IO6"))
 (segment (start 99.9004 75.0995) (end 99.9001 75.0998) (width 1) (layer "F.Cu") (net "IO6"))
 (segment (start 99.9001 75.0998) (end 99.9001 75.9999) (width 1) (layer "F.Cu") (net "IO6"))
 (segment (start 101.3004 77.1396) (end 90.71 87.73) (width 1) (layer "F.Cu") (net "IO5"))
 (segment (start 101.3004 75.0998) (end 101.3004 77.1396) (width 1) (layer "F.Cu") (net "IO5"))
 (segment (start 102.6999 78.2801) (end 90.71 90.27) (width 1) (layer "F.Cu") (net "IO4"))
 (segment (start 90.77 90.33) (end 90.71 90.27) (width 1) (layer "F.Cu") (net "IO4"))
 (segment (start 102.6999 75.0998) (end 102.6999 78.2801) (width 1) (layer "F.Cu") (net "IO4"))
 (segment (start 104.1 75.0998) (end 104.1 79.42) (width 1) (layer "F.Cu") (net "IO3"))
 (segment (start 104.1 75.0998) (end 104.0999 75.0998) (width 1) (layer "F.Cu") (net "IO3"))
 (segment (start 104.1 79.42) (end 90.71 92.81) (width 1) (layer "F.Cu") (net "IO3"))
 (segment (start 114.4001 65.7001) (end 111.75051 65.7001) (width 1) (layer "F.Cu") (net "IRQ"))
 (segment (start 118.65 69.95) (end 114.4001 65.7001) (width 1) (layer "F.Cu") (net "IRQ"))
 (segment (start 116.19 72.57) (end 116.19 70.380203) (width 1) (layer "F.Cu") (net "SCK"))
 (segment (start 118.65 75.03) (end 118.59 75.09) (width 1) (layer "F.Cu") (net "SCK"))
 (segment (start 114.309697 68.4999) (end 111.1 68.4999) (width 1) (layer "F.Cu") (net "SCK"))
 (segment (start 118.65 75.03) (end 116.19 72.57) (width 1) (layer "F.Cu") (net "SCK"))
 (segment (start 116.19 70.380203) (end 114.309697 68.4999) (width 1) (layer "F.Cu") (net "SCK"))
 (segment (start 118.65 77.57) (end 114.55 73.47) (width 1) (layer "F.Cu") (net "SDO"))
 (segment (start 114.55 70.720101) (end 113.729799 69.8999) (width 1) (layer "F.Cu") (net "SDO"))
 (segment (start 114.55 73.47) (end 114.55 70.720101) (width 1) (layer "F.Cu") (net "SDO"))
 (segment (start 113.729799 69.8999) (end 111.1 69.8999) (width 1) (layer "F.Cu") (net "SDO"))
 (segment (start 111.1001 71.2999) (end 111.1 71.3) (width 1) (layer "F.Cu") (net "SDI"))
 (segment (start 118.65 80.11) (end 113.15 74.61) (width 1) (layer "F.Cu") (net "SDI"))
 (segment (start 113.15 71.3) (end 111.1 71.3) (width 1) (layer "F.Cu") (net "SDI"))
 (segment (start 113.15 74.61) (end 113.15 71.3) (width 1) (layer "F.Cu") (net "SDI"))
 (segment (start 118.65 82.65) (end 111.1 75.1) (width 1) (layer "F.Cu") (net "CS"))
 (segment (start 111.1 75.1) (end 111.1 72.7) (width 1) (layer "F.Cu") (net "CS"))
 (segment (start 108.405 75.2044) (end 108.3004 75.0998) (width 0.4) (layer "F.Cu") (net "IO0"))
 (segment (start 108.3004 77.3804) (end 108.3004 75.0998) (width 1) (layer "F.Cu") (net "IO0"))
 (segment (start 118.65 87.73) (end 108.3004 77.3804) (width 1) (layer "F.Cu") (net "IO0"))
 (segment (start 106.9001 78.5201) (end 106.9001 75.0998) (width 1) (layer "F.Cu") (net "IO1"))
 (segment (start 118.65 90.27) (end 106.9001 78.5201) (width 1) (layer "F.Cu") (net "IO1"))
 (segment (start 118.65 92.81) (end 105.5 79.66) (width 1) (layer "F.Cu") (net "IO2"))
 (segment (start 105.5 79.66) (end 105.5 75.0998) (width 1) (layer "F.Cu") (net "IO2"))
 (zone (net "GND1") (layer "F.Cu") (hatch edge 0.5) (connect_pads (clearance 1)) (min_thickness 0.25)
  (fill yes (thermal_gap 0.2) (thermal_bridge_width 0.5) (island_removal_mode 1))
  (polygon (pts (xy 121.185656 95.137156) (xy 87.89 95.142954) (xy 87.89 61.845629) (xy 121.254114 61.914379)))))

